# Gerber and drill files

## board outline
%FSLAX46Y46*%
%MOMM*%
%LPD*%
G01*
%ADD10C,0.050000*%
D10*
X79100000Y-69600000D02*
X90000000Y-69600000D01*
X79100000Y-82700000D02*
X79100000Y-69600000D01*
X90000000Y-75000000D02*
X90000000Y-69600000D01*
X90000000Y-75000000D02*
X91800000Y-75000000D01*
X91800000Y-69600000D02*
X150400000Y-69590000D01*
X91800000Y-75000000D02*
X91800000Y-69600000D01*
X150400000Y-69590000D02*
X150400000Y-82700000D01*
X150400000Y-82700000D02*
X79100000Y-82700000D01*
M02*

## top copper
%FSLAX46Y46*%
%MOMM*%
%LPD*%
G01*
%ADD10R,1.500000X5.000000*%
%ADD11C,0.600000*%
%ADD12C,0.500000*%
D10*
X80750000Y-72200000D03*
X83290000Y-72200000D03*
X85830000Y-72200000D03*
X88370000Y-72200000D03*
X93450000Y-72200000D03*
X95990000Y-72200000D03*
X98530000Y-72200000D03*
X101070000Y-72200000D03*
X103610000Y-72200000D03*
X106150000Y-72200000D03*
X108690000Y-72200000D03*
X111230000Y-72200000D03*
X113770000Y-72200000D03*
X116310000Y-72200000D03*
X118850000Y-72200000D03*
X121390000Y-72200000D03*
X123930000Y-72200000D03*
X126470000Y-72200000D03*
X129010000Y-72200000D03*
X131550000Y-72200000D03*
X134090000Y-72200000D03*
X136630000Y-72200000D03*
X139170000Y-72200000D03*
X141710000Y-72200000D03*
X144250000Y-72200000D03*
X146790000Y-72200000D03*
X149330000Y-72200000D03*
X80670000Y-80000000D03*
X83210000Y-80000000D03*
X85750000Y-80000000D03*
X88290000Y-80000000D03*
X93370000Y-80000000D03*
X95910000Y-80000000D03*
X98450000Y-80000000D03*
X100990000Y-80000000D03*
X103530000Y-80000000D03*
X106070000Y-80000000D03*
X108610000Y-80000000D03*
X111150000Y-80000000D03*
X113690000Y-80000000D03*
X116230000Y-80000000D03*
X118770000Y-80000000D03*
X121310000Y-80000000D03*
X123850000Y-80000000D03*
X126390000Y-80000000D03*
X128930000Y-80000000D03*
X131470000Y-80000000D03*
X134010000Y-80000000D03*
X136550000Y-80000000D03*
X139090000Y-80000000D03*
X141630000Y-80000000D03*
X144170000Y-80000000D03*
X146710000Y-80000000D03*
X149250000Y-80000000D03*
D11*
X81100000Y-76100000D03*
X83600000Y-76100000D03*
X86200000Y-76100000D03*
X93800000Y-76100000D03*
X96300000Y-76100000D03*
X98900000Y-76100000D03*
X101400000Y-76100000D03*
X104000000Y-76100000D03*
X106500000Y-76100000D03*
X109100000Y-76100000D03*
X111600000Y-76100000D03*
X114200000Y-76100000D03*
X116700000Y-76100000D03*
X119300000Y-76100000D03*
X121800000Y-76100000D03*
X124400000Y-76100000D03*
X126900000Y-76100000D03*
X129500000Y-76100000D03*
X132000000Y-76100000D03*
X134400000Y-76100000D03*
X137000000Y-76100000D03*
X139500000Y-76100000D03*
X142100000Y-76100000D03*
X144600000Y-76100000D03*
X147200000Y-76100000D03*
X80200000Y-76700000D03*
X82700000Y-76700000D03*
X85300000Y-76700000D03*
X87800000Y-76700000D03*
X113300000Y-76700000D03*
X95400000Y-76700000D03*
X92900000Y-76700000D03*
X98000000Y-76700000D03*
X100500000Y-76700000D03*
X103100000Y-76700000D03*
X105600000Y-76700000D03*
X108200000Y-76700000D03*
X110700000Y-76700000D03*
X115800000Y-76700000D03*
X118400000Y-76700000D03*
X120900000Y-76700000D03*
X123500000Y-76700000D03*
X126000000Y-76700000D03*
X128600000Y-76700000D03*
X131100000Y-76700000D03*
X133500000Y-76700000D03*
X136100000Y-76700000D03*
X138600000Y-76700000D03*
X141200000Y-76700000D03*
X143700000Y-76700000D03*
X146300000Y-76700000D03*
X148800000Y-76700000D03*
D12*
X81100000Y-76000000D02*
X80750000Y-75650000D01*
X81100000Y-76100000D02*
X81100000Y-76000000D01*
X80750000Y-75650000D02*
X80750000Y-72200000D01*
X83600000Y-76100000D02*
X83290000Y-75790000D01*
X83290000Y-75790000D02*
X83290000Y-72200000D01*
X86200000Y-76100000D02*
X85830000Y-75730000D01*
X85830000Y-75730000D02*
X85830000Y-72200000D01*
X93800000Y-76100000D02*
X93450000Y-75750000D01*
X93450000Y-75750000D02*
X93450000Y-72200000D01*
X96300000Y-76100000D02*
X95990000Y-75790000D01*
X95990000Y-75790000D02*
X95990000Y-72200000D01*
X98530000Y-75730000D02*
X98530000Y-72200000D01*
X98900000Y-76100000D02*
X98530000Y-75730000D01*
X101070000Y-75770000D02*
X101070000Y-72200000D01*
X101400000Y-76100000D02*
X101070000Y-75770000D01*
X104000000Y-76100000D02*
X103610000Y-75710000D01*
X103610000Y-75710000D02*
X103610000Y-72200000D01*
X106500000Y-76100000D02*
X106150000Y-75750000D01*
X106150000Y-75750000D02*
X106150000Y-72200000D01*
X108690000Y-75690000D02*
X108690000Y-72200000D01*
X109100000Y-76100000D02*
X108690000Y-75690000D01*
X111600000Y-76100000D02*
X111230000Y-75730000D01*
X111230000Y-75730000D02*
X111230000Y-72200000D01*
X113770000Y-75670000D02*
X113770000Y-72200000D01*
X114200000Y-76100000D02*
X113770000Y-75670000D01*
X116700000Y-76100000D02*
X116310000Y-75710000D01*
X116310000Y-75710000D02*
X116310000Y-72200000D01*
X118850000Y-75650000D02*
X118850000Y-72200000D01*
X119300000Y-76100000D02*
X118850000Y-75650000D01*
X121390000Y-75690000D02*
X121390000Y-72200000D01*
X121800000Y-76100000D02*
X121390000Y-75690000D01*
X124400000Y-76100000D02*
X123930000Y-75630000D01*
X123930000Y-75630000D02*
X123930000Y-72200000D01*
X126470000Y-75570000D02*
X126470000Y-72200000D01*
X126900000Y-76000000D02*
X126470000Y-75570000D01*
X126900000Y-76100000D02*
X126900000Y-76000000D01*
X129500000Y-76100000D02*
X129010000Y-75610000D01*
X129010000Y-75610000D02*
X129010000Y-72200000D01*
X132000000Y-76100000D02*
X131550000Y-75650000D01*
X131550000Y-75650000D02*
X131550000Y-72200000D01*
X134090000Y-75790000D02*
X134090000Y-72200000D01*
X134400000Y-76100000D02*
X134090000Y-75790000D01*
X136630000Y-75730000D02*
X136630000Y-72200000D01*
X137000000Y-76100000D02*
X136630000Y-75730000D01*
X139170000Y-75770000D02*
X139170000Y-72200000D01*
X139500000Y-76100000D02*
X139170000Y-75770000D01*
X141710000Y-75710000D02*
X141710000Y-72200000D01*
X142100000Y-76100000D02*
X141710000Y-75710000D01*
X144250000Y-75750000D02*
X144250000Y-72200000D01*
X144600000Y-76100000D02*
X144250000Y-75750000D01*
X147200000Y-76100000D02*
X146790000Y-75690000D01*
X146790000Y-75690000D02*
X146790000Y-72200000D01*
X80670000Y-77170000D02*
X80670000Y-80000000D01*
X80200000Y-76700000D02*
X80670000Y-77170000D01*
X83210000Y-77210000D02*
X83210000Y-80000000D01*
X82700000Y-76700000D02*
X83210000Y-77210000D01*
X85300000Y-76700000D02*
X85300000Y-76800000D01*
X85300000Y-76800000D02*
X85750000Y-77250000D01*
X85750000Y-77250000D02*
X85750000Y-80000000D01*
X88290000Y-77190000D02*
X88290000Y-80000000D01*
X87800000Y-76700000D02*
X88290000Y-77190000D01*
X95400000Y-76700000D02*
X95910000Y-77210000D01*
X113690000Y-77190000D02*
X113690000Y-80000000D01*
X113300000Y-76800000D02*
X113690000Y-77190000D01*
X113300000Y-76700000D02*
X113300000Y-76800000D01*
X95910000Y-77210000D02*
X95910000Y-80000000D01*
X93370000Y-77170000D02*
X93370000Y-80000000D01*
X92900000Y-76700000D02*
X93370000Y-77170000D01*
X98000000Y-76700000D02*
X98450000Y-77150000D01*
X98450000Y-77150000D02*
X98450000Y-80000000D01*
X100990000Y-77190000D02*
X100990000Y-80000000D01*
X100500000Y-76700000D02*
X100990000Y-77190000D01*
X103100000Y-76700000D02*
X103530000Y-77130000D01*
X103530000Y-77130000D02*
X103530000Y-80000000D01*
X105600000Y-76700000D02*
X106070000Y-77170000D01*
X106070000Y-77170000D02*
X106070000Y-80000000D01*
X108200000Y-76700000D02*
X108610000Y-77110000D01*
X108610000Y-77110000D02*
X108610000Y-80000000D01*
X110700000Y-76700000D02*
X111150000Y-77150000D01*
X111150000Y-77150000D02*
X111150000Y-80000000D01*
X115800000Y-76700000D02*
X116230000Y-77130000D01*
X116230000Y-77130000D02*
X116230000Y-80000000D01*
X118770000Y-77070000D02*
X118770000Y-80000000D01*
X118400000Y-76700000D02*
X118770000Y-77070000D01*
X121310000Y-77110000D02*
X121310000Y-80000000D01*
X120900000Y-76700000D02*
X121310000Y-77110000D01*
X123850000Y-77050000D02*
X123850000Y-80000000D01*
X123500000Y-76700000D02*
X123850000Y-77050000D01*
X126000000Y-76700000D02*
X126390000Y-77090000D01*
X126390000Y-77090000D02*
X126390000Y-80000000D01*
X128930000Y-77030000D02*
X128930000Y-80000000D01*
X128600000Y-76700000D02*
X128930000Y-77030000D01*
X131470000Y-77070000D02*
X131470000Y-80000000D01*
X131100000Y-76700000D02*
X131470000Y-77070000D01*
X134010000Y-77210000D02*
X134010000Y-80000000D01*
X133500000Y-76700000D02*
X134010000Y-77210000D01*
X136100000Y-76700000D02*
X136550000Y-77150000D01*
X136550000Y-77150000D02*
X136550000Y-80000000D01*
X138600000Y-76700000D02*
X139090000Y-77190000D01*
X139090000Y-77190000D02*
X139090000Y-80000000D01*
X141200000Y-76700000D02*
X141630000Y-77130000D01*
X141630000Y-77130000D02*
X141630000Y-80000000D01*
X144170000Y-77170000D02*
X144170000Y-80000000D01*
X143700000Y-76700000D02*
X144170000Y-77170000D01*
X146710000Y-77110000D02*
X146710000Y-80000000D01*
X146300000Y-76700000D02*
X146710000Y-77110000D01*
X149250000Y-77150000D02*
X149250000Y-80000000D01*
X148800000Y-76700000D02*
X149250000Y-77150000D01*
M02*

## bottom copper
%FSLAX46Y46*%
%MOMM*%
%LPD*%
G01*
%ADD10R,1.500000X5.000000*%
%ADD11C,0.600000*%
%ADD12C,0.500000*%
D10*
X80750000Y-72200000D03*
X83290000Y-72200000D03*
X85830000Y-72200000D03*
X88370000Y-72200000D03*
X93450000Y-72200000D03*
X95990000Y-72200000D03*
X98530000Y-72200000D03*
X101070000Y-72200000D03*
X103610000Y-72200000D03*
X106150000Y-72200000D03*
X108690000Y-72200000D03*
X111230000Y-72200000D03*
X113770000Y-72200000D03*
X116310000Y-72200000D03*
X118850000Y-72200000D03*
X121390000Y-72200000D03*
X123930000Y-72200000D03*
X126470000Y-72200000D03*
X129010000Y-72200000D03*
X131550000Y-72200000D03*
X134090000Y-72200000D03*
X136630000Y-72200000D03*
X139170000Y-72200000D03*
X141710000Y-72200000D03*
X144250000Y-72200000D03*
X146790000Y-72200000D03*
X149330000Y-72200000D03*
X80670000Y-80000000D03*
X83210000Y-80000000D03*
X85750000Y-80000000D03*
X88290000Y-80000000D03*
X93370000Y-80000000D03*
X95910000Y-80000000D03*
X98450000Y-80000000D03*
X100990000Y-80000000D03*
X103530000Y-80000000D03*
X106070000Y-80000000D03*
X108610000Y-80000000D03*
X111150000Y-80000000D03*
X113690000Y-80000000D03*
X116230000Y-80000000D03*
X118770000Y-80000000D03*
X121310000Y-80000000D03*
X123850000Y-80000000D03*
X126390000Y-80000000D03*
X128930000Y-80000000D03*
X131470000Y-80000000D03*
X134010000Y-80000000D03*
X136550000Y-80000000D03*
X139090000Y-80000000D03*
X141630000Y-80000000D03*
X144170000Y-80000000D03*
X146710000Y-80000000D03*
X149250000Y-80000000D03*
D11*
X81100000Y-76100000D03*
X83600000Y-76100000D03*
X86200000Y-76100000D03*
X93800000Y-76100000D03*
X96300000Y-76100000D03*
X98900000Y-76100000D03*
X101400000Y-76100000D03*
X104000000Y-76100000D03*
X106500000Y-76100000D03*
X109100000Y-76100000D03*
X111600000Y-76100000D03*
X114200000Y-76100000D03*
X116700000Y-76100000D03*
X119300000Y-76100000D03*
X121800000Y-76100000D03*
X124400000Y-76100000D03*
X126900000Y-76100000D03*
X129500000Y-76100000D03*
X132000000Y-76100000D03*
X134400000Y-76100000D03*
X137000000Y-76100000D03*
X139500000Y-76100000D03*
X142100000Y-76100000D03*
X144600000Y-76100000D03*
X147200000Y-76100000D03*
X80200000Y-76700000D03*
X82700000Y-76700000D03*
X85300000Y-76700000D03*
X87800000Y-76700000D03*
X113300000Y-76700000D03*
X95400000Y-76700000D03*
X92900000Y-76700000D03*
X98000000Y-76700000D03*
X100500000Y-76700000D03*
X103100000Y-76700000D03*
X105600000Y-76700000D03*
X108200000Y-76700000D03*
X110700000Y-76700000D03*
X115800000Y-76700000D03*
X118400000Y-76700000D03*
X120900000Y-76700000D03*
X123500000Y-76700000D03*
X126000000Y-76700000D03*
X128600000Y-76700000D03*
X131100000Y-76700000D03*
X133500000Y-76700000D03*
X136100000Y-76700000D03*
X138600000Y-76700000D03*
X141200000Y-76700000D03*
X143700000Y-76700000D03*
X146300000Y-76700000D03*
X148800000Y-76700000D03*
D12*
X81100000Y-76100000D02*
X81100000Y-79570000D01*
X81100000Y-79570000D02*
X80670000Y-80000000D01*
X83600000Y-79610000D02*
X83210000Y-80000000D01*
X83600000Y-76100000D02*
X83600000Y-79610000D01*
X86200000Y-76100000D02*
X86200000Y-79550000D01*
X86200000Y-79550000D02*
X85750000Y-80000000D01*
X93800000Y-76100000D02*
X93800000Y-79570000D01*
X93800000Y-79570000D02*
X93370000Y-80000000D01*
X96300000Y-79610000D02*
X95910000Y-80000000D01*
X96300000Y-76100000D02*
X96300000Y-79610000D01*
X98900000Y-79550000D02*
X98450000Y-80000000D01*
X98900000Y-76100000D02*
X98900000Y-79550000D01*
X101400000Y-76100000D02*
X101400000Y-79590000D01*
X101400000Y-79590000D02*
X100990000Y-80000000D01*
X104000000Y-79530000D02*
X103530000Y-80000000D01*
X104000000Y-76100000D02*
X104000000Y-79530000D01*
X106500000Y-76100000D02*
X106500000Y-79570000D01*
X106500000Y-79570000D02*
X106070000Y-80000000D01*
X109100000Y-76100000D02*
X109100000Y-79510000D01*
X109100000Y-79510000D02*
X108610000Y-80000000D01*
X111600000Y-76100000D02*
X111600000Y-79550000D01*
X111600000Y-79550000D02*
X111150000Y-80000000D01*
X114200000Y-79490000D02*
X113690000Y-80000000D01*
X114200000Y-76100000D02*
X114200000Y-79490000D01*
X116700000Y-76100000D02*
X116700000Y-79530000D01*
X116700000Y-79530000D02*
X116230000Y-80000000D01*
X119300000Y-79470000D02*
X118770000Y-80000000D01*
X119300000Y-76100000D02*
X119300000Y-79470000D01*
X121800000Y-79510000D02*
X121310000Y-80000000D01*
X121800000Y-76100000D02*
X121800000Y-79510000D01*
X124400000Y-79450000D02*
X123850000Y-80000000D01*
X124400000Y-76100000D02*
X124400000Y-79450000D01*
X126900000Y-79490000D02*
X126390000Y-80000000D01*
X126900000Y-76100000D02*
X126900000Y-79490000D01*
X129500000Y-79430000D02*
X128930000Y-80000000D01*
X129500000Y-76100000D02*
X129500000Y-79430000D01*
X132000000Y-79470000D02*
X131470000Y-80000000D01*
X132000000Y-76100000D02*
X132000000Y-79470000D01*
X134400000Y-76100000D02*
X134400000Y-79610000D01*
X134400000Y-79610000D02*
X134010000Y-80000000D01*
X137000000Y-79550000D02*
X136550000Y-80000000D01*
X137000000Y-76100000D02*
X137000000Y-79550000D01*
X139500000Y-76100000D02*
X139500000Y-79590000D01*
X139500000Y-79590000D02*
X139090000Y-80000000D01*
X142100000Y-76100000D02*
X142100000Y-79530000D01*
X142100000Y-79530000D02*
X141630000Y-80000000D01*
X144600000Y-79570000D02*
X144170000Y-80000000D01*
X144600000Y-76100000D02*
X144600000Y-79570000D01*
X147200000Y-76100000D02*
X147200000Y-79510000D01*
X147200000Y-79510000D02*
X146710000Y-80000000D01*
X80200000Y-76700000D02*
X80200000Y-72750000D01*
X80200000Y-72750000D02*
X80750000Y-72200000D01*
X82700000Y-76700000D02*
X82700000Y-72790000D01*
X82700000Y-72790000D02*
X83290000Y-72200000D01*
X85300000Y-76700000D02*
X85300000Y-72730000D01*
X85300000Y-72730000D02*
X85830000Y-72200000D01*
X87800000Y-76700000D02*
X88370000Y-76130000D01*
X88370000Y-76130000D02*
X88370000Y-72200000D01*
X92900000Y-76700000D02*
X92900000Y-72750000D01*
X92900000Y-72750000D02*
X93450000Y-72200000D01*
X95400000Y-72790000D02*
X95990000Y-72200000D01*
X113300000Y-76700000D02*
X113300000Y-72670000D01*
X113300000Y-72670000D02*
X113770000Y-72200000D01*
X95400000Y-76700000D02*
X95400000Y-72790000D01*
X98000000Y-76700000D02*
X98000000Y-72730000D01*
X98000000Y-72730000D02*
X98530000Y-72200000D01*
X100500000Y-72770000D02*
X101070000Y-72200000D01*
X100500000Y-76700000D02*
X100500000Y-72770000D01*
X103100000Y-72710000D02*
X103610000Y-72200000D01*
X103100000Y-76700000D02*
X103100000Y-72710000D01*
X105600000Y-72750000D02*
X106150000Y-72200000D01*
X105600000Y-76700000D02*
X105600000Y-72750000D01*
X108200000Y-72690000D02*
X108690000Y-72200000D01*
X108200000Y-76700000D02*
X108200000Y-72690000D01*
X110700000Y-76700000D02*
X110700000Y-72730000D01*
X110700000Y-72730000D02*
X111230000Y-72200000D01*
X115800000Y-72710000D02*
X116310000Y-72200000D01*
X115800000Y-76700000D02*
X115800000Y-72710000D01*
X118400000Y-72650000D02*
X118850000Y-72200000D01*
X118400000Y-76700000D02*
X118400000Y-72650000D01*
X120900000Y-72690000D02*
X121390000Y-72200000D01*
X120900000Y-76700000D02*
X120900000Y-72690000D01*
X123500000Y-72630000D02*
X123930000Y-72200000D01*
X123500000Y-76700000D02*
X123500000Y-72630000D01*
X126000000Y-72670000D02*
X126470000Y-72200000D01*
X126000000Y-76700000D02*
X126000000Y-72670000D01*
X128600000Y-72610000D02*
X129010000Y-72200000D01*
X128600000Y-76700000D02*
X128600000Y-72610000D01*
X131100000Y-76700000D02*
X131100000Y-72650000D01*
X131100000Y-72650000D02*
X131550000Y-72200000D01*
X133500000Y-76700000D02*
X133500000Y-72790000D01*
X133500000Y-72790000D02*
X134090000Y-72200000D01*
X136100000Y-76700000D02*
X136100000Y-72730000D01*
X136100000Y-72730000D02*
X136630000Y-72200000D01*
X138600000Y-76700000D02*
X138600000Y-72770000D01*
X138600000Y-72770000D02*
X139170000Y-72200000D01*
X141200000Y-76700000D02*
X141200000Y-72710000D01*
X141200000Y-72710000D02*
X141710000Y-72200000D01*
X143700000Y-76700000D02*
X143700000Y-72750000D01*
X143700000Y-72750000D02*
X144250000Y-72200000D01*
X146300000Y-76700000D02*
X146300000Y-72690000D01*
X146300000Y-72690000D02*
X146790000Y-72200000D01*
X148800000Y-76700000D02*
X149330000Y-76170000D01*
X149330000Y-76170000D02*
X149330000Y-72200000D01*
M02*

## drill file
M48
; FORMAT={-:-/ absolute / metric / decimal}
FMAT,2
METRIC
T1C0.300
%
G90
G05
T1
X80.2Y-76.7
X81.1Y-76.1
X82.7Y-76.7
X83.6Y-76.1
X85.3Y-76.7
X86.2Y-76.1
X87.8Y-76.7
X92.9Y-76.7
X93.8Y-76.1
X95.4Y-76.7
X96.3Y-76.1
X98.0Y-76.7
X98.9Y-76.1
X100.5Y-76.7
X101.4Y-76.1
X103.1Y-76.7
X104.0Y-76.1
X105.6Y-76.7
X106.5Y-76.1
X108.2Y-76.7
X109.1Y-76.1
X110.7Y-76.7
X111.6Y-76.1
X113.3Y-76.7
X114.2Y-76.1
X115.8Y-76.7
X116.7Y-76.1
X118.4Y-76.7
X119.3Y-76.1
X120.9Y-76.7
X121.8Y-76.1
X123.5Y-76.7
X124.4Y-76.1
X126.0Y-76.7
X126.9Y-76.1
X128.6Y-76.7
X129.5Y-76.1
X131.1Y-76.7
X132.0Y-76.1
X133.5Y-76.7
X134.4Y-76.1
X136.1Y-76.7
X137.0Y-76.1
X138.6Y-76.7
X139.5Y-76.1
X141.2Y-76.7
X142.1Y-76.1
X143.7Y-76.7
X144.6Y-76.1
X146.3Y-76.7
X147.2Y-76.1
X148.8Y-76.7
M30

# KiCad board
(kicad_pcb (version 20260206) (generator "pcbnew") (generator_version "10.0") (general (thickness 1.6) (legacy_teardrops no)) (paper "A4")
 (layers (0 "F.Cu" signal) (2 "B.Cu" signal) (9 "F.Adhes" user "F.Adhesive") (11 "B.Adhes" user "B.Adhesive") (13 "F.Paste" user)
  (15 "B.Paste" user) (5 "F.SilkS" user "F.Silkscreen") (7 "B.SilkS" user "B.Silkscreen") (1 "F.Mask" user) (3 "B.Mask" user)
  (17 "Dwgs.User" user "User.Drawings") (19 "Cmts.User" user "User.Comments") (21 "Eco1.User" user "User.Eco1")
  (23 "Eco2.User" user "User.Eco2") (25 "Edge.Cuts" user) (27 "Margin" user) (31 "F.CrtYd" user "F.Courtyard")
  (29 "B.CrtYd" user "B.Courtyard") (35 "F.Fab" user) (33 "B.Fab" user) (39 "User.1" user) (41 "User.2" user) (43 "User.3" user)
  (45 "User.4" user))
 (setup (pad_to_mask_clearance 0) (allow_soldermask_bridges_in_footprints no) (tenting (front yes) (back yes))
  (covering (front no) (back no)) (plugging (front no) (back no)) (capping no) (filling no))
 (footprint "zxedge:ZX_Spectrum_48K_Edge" (layer "F.Cu") (at 115.04 74.7)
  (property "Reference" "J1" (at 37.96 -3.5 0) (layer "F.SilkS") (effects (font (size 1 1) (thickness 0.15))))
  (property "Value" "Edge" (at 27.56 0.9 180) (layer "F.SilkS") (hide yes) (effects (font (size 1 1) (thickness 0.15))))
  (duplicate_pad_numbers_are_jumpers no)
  (pad "A1" smd rect (at -34.29 -2.5) (size 1.5 5) (layers "F.Cu" "F.Mask") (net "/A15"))
  (pad "A2" smd rect (at -31.75 -2.5) (size 1.5 5) (layers "F.Cu" "F.Mask") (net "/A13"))
  (pad "A3" smd rect (at -29.21 -2.5) (size 1.5 5) (layers "F.Cu" "F.Mask") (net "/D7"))
  (pad "A4" smd rect (at -26.67 -2.5) (size 1.5 5) (layers "F.Cu" "F.Mask") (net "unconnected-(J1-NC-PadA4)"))
  (pad "A6" smd rect (at -21.59 -2.5) (size 1.5 5) (layers "F.Cu" "F.Mask") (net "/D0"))
  (pad "A7" smd rect (at -19.05 -2.5) (size 1.5 5) (layers "F.Cu" "F.Mask") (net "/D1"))
  (pad "A8" smd rect (at -16.51 -2.5) (size 1.5 5) (layers "F.Cu" "F.Mask") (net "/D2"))
  (pad "A9" smd rect (at -13.97 -2.5) (size 1.5 5) (layers "F.Cu" "F.Mask") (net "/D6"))
  (pad "A10" smd rect (at -11.43 -2.5) (size 1.5 5) (layers "F.Cu" "F.Mask") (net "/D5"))
  (pad "A11" smd rect (at -8.89 -2.5) (size 1.5 5) (layers "F.Cu" "F.Mask") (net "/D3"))
  (pad "A12" smd rect (at -6.35 -2.5) (size 1.5 5) (layers "F.Cu" "F.Mask") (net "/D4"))
  (pad "A13" smd rect (at -3.81 -2.5) (size 1.5 5) (layers "F.Cu" "F.Mask") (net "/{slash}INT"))
  (pad "A14" smd rect (at -1.27 -2.5) (size 1.5 5) (layers "F.Cu" "F.Mask") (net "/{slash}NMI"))
  (pad "A15" smd rect (at 1.27 -2.5) (size 1.5 5) (layers "F.Cu" "F.Mask") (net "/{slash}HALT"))
  (pad "A16" smd rect (at 3.81 -2.5) (size 1.5 5) (layers "F.Cu" "F.Mask") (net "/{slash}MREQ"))
  (pad "A17" smd rect (at 6.35 -2.5) (size 1.5 5) (layers "F.Cu" "F.Mask") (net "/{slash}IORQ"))
  (pad "A18" smd rect (at 8.89 -2.5) (size 1.5 5) (layers "F.Cu" "F.Mask") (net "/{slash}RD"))
  (pad "A19" smd rect (at 11.43 -2.5) (size 1.5 5) (layers "F.Cu" "F.Mask") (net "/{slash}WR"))
  (pad "A20" smd rect (at 13.97 -2.5) (size 1.5 5) (layers "F.Cu" "F.Mask") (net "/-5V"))
  (pad "A21" smd rect (at 16.51 -2.5) (size 1.5 5) (layers "F.Cu" "F.Mask") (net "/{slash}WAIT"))
  (pad "A22" smd rect (at 19.05 -2.5) (size 1.5 5) (layers "F.Cu" "F.Mask") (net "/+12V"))
  (pad "A23" smd rect (at 21.59 -2.5) (size 1.5 5) (layers "F.Cu" "F.Mask") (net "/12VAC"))
  (pad "A24" smd rect (at 24.13 -2.5) (size 1.5 5) (layers "F.Cu" "F.Mask") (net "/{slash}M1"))
  (pad "A25" smd rect (at 26.67 -2.5) (size 1.5 5) (layers "F.Cu" "F.Mask") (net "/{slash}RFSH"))
  (pad "A26" smd rect (at 29.21 -2.5) (size 1.5 5) (layers "F.Cu" "F.Mask") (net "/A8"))
  (pad "A27" smd rect (at 31.75 -2.5) (size 1.5 5) (layers "F.Cu" "F.Mask") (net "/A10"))
  (pad "A28" smd rect (at 34.29 -2.5) (size 1.5 5) (layers "F.Cu" "F.Mask") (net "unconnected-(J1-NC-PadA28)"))
  (pad "B1" smd rect (at -34.29 -2.5) (size 1.5 5) (layers "B.Cu" "B.Mask") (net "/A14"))
  (pad "B2" smd rect (at -31.75 -2.5) (size 1.5 5) (layers "B.Cu" "B.Mask") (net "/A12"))
  (pad "B3" smd rect (at -29.21 -2.5) (size 1.5 5) (layers "B.Cu" "B.Mask") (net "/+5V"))
  (pad "B4" smd rect (at -26.67 -2.5) (size 1.5 5) (layers "B.Cu" "B.Mask") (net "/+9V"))
  (pad "B6" smd rect (at -21.59 -2.5) (size 1.5 5) (layers "B.Cu" "B.Mask") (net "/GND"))
  (pad "B7" smd rect (at -19.05 -2.5) (size 1.5 5) (layers "B.Cu" "B.Mask") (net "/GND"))
  (pad "B8" smd rect (at -16.51 -2.5) (size 1.5 5) (layers "B.Cu" "B.Mask") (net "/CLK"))
  (pad "B9" smd rect (at -13.97 -2.5) (size 1.5 5) (layers "B.Cu" "B.Mask") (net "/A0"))
  (pad "B10" smd rect (at -11.43 -2.5) (size 1.5 5) (layers "B.Cu" "B.Mask") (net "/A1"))
  (pad "B11" smd rect (at -8.89 -2.5) (size 1.5 5) (layers "B.Cu" "B.Mask") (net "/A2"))
  (pad "B12" smd rect (at -6.35 -2.5) (size 1.5 5) (layers "B.Cu" "B.Mask") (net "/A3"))
  (pad "B13" smd rect (at -3.81 -2.5) (size 1.5 5) (layers "B.Cu" "B.Mask") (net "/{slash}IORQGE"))
  (pad "B14" smd rect (at -1.27 -2.5) (size 1.5 5) (layers "B.Cu" "B.Mask") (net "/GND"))
  (pad "B15" smd rect (at 1.27 -2.5) (size 1.5 5) (layers "B.Cu" "B.Mask") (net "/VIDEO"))
  (pad "B16" smd rect (at 3.81 -2.5) (size 1.5 5) (layers "B.Cu" "B.Mask") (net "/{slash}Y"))
  (pad "B17" smd rect (at 6.35 -2.5) (size 1.5 5) (layers "B.Cu" "B.Mask") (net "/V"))
  (pad "B18" smd rect (at 8.89 -2.5) (size 1.5 5) (layers "B.Cu" "B.Mask") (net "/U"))
  (pad "B19" smd rect (at 11.43 -2.5) (size 1.5 5) (layers "B.Cu" "B.Mask") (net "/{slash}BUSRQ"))
  (pad "B20" smd rect (at 13.97 -2.5) (size 1.5 5) (layers "B.Cu" "B.Mask") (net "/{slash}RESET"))
  (pad "B21" smd rect (at 16.51 -2.5) (size 1.5 5) (layers "B.Cu" "B.Mask") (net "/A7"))
  (pad "B22" smd rect (at 19.05 -2.5) (size 1.5 5) (layers "B.Cu" "B.Mask") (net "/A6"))
  (pad "B23" smd rect (at 21.59 -2.5) (size 1.5 5) (layers "B.Cu" "B.Mask") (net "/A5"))
  (pad "B24" smd rect (at 24.13 -2.5) (size 1.5 5) (layers "B.Cu" "B.Mask") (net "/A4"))
  (pad "B25" smd rect (at 26.67 -2.5) (size 1.5 5) (layers "B.Cu" "B.Mask") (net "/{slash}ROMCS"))
  (pad "B26" smd rect (at 29.21 -2.5) (size 1.5 5) (layers "B.Cu" "B.Mask") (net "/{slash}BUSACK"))
  (pad "B27" smd rect (at 31.75 -2.5) (size 1.5 5) (layers "B.Cu" "B.Mask") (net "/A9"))
  (pad "B28" smd rect (at 34.29 -2.5) (size 1.5 5) (layers "B.Cu" "B.Mask") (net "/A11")))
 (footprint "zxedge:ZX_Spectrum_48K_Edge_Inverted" (layer "B.Cu") (at 114.96 77.5)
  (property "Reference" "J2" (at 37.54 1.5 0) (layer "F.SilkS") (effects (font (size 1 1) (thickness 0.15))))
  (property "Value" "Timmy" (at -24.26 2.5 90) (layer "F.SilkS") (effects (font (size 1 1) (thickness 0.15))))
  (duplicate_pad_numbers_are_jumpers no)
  (pad "A1" smd rect (at -34.29 2.5) (size 1.5 5) (layers "F.Cu" "F.Mask") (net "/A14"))
  (pad "A2" smd rect (at -31.75 2.5) (size 1.5 5) (layers "F.Cu" "F.Mask") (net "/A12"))
  (pad "A3" smd rect (at -29.21 2.5) (size 1.5 5) (layers "F.Cu" "F.Mask") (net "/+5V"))
  (pad "A4" smd rect (at -26.67 2.5) (size 1.5 5) (layers "F.Cu" "F.Mask") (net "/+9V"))
  (pad "A6" smd rect (at -21.59 2.5) (size 1.5 5) (layers "F.Cu" "F.Mask") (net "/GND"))
  (pad "A7" smd rect (at -19.05 2.5) (size 1.5 5) (layers "F.Cu" "F.Mask") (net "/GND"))
  (pad "A8" smd rect (at -16.51 2.5) (size 1.5 5) (layers "F.Cu" "F.Mask") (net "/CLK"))
  (pad "A9" smd rect (at -13.97 2.5) (size 1.5 5) (layers "F.Cu" "F.Mask") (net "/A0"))
  (pad "A10" smd rect (at -11.43 2.5) (size 1.5 5) (layers "F.Cu" "F.Mask") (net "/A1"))
  (pad "A11" smd rect (at -8.89 2.5) (size 1.5 5) (layers "F.Cu" "F.Mask") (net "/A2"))
  (pad "A12" smd rect (at -6.35 2.5) (size 1.5 5) (layers "F.Cu" "F.Mask") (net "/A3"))
  (pad "A13" smd rect (at -3.81 2.5) (size 1.5 5) (layers "F.Cu" "F.Mask") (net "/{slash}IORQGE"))
  (pad "A14" smd rect (at -1.27 2.5) (size 1.5 5) (layers "F.Cu" "F.Mask") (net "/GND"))
  (pad "A15" smd rect (at 1.27 2.5) (size 1.5 5) (layers "F.Cu" "F.Mask") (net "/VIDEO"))
  (pad "A16" smd rect (at 3.81 2.5) (size 1.5 5) (layers "F.Cu" "F.Mask") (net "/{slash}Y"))
  (pad "A17" smd rect (at 6.35 2.5) (size 1.5 5) (layers "F.Cu" "F.Mask") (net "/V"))
  (pad "A18" smd rect (at 8.89 2.5) (size 1.5 5) (layers "F.Cu" "F.Mask") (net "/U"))
  (pad "A19" smd rect (at 11.43 2.5) (size 1.5 5) (layers "F.Cu" "F.Mask") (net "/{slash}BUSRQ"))
  (pad "A20" smd rect (at 13.97 2.5) (size 1.5 5) (layers "F.Cu" "F.Mask") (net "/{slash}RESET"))
  (pad "A21" smd rect (at 16.51 2.5) (size 1.5 5) (layers "F.Cu" "F.Mask") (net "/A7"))
  (pad "A22" smd rect (at 19.05 2.5) (size 1.5 5) (layers "F.Cu" "F.Mask") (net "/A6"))
  (pad "A23" smd rect (at 21.59 2.5) (size 1.5 5) (layers "F.Cu" "F.Mask") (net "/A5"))
  (pad "A24" smd rect (at 24.13 2.5) (size 1.5 5) (layers "F.Cu" "F.Mask") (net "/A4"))
  (pad "A25" smd rect (at 26.67 2.5) (size 1.5 5) (layers "F.Cu" "F.Mask") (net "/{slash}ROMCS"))
  (pad "A26" smd rect (at 29.21 2.5) (size 1.5 5) (layers "F.Cu" "F.Mask") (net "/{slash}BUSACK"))
  (pad "A27" smd rect (at 31.75 2.5) (size 1.5 5) (layers "F.Cu" "F.Mask") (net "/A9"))
  (pad "A28" smd rect (at 34.29 2.5) (size 1.5 5) (layers "F.Cu" "F.Mask") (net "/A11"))
  (pad "B1" smd rect (at -34.29 2.5) (size 1.5 5) (layers "B.Cu" "B.Mask") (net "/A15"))
  (pad "B2" smd rect (at -31.75 2.5) (size 1.5 5) (layers "B.Cu" "B.Mask") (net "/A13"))
  (pad "B3" smd rect (at -29.21 2.5) (size 1.5 5) (layers "B.Cu" "B.Mask") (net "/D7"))
  (pad "B4" smd rect (at -26.67 2.5) (size 1.5 5) (layers "B.Cu" "B.Mask") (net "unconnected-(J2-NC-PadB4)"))
  (pad "B6" smd rect (at -21.59 2.5) (size 1.5 5) (layers "B.Cu" "B.Mask") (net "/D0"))
  (pad "B7" smd rect (at -19.05 2.5) (size 1.5 5) (layers "B.Cu" "B.Mask") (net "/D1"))
  (pad "B8" smd rect (at -16.51 2.5) (size 1.5 5) (layers "B.Cu" "B.Mask") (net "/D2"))
  (pad "B9" smd rect (at -13.97 2.5) (size 1.5 5) (layers "B.Cu" "B.Mask") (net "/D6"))
  (pad "B10" smd rect (at -11.43 2.5) (size 1.5 5) (layers "B.Cu" "B.Mask") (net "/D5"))
  (pad "B11" smd rect (at -8.89 2.5) (size 1.5 5) (layers "B.Cu" "B.Mask") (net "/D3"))
  (pad "B12" smd rect (at -6.35 2.5) (size 1.5 5) (layers "B.Cu" "B.Mask") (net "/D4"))
  (pad "B13" smd rect (at -3.81 2.5) (size 1.5 5) (layers "B.Cu" "B.Mask") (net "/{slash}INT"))
  (pad "B14" smd rect (at -1.27 2.5) (size 1.5 5) (layers "B.Cu" "B.Mask") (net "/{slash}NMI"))
  (pad "B15" smd rect (at 1.27 2.5) (size 1.5 5) (layers "B.Cu" "B.Mask") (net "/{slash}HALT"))
  (pad "B16" smd rect (at 3.81 2.5) (size 1.5 5) (layers "B.Cu" "B.Mask") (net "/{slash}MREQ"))
  (pad "B17" smd rect (at 6.35 2.5) (size 1.5 5) (layers "B.Cu" "B.Mask") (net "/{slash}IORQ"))
  (pad "B18" smd rect (at 8.89 2.5) (size 1.5 5) (layers "B.Cu" "B.Mask") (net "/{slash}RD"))
  (pad "B19" smd rect (at 11.43 2.5) (size 1.5 5) (layers "B.Cu" "B.Mask") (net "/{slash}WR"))
  (pad "B20" smd rect (at 13.97 2.5) (size 1.5 5) (layers "B.Cu" "B.Mask") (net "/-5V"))
  (pad "B21" smd rect (at 16.51 2.5) (size 1.5 5) (layers "B.Cu" "B.Mask") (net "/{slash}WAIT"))
  (pad "B22" smd rect (at 19.05 2.5) (size 1.5 5) (layers "B.Cu" "B.Mask") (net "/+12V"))
  (pad "B23" smd rect (at 21.59 2.5) (size 1.5 5) (layers "B.Cu" "B.Mask") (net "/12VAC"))
  (pad "B24" smd rect (at 24.13 2.5) (size 1.5 5) (layers "B.Cu" "B.Mask") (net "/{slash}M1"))
  (pad "B25" smd rect (at 26.67 2.5) (size 1.5 5) (layers "B.Cu" "B.Mask") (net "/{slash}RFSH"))
  (pad "B26" smd rect (at 29.21 2.5) (size 1.5 5) (layers "B.Cu" "B.Mask") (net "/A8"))
  (pad "B27" smd rect (at 31.75 2.5) (size 1.5 5) (layers "B.Cu" "B.Mask") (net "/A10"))
  (pad "B28" smd rect (at 34.29 2.5) (size 1.5 5) (layers "B.Cu" "B.Mask") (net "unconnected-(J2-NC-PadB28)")))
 (gr_line (start 79.1 69.6) (end 90 69.6) (stroke (width 0.05) (type default)) (layer "Edge.Cuts"))
 (gr_line (start 79.1 82.7) (end 79.1 69.6) (stroke (width 0.05) (type default)) (layer "Edge.Cuts"))
 (gr_line (start 90 75) (end 90 69.6) (stroke (width 0.05) (type default)) (layer "Edge.Cuts"))
 (gr_line (start 90 75) (end 91.8 75) (stroke (width 0.05) (type default)) (layer "Edge.Cuts"))
 (gr_line (start 91.8 69.6) (end 150.4 69.59) (stroke (width 0.05) (type default)) (layer "Edge.Cuts"))
 (gr_line (start 91.8 75) (end 91.8 69.6) (stroke (width 0.05) (type default)) (layer "Edge.Cuts"))
 (gr_line (start 150.4 69.59) (end 150.4 82.7) (stroke (width 0.05) (type default)) (layer "Edge.Cuts"))
 (gr_line (start 150.4 82.7) (end 79.1 82.7) (stroke (width 0.05) (type default)) (layer "Edge.Cuts"))
 (segment (start 81.1 76) (end 80.75 75.65) (width 0.5) (layer "F.Cu") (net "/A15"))
 (segment (start 81.1 76.1) (end 81.1 76) (width 0.5) (layer "F.Cu") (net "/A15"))
 (segment (start 80.75 75.65) (end 80.75 72.2) (width 0.5) (layer "F.Cu") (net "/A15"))
 (via (at 81.1 76.1) (size 0.6) (drill 0.3) (layers "F.Cu" "B.Cu") (free yes) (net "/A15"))
 (segment (start 81.1 76.1) (end 81.1 79.57) (width 0.5) (layer "B.Cu") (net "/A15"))
 (segment (start 81.1 79.57) (end 80.67 80) (width 0.5) (layer "B.Cu") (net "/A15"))
 (segment (start 83.6 76.1) (end 83.29 75.79) (width 0.5) (layer "F.Cu") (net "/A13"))
 (segment (start 83.29 75.79) (end 83.29 72.2) (width 0.5) (layer "F.Cu") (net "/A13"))
 (via (at 83.6 76.1) (size 0.6) (drill 0.3) (layers "F.Cu" "B.Cu") (free yes) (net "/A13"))
 (segment (start 83.6 79.61) (end 83.21 80) (width 0.5) (layer "B.Cu") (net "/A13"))
 (segment (start 83.6 76.1) (end 83.6 79.61) (width 0.5) (layer "B.Cu") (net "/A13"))
 (segment (start 86.2 76.1) (end 85.83 75.73) (width 0.5) (layer "F.Cu") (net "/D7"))
 (segment (start 85.83 75.73) (end 85.83 72.2) (width 0.5) (layer "F.Cu") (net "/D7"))
 (via (at 86.2 76.1) (size 0.6) (drill 0.3) (layers "F.Cu" "B.Cu") (free yes) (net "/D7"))
 (segment (start 86.2 76.1) (end 86.2 79.55) (width 0.5) (layer "B.Cu") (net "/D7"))
 (segment (start 86.2 79.55) (end 85.75 80) (width 0.5) (layer "B.Cu") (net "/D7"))
 (segment (start 93.8 76.1) (end 93.45 75.75) (width 0.5) (layer "F.Cu") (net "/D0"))
 (segment (start 93.45 75.75) (end 93.45 72.2) (width 0.5) (layer "F.Cu") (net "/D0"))
 (via (at 93.8 76.1) (size 0.6) (drill 0.3) (layers "F.Cu" "B.Cu") (free yes) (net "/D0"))
 (segment (start 93.8 76.1) (end 93.8 79.57) (width 0.5) (layer "B.Cu") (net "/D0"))
 (segment (start 93.8 79.57) (end 93.37 80) (width 0.5) (layer "B.Cu") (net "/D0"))
 (segment (start 96.3 76.1) (end 95.99 75.79) (width 0.5) (layer "F.Cu") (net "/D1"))
 (segment (start 95.99 75.79) (end 95.99 72.2) (width 0.5) (layer "F.Cu") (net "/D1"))
 (via (at 96.3 76.1) (size 0.6) (drill 0.3) (layers "F.Cu" "B.Cu") (free yes) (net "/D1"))
 (segment (start 96.3 79.61) (end 95.91 80) (width 0.5) (layer "B.Cu") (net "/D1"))
 (segment (start 96.3 76.1) (end 96.3 79.61) (width 0.5) (layer "B.Cu") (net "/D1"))
 (segment (start 98.53 75.73) (end 98.53 72.2) (width 0.5) (layer "F.Cu") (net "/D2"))
 (segment (start 98.9 76.1) (end 98.53 75.73) (width 0.5) (layer "F.Cu") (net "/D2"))
 (via (at 98.9 76.1) (size 0.6) (drill 0.3) (layers "F.Cu" "B.Cu") (free yes) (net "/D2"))
 (segment (start 98.9 79.55) (end 98.45 80) (width 0.5) (layer "B.Cu") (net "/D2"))
 (segment (start 98.9 76.1) (end 98.9 79.55) (width 0.5) (layer "B.Cu") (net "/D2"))
 (segment (start 101.07 75.77) (end 101.07 72.2) (width 0.5) (layer "F.Cu") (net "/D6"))
 (segment (start 101.4 76.1) (end 101.07 75.77) (width 0.5) (layer "F.Cu") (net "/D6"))
 (via (at 101.4 76.1) (size 0.6) (drill 0.3) (layers "F.Cu" "B.Cu") (free yes) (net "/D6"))
 (segment (start 101.4 76.1) (end 101.4 79.59) (width 0.5) (layer "B.Cu") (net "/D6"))
 (segment (start 101.4 79.59) (end 100.99 80) (width 0.5) (layer "B.Cu") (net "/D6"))
 (segment (start 104 76.1) (end 103.61 75.71) (width 0.5) (layer "F.Cu") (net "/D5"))
 (segment (start 103.61 75.71) (end 103.61 72.2) (width 0.5) (layer "F.Cu") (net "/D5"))
 (via (at 104 76.1) (size 0.6) (drill 0.3) (layers "F.Cu" "B.Cu") (free yes) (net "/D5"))
 (segment (start 104 79.53) (end 103.53 80) (width 0.5) (layer "B.Cu") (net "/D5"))
 (segment (start 104 76.1) (end 104 79.53) (width 0.5) (layer "B.Cu") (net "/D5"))
 (segment (start 106.5 76.1) (end 106.15 75.75) (width 0.5) (layer "F.Cu") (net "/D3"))
 (segment (start 106.15 75.75) (end 106.15 72.2) (width 0.5) (layer "F.Cu") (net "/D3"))
 (via (at 106.5 76.1) (size 0.6) (drill 0.3) (layers "F.Cu" "B.Cu") (free yes) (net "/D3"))
 (segment (start 106.5 76.1) (end 106.5 79.57) (width 0.5) (layer "B.Cu") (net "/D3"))
 (segment (start 106.5 79.57) (end 106.07 80) (width 0.5) (layer "B.Cu") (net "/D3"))
 (segment (start 108.69 75.69) (end 108.69 72.2) (width 0.5) (layer "F.Cu") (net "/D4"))
 (segment (start 109.1 76.1) (end 108.69 75.69) (width 0.5) (layer "F.Cu") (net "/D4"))
 (via (at 109.1 76.1) (size 0.6) (drill 0.3) (layers "F.Cu" "B.Cu") (free yes) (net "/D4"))
 (segment (start 109.1 76.1) (end 109.1 79.51) (width 0.5) (layer "B.Cu") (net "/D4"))
 (segment (start 109.1 79.51) (end 108.61 80) (width 0.5) (layer "B.Cu") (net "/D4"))
 (segment (start 111.6 76.1) (end 111.23 75.73) (width 0.5) (layer "F.Cu") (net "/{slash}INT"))
 (segment (start 111.23 75.73) (end 111.23 72.2) (width 0.5) (layer "F.Cu") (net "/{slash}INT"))
 (via (at 111.6 76.1) (size 0.6) (drill 0.3) (layers "F.Cu" "B.Cu") (free yes) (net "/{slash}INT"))
 (segment (start 111.6 76.1) (end 111.6 79.55) (width 0.5) (layer "B.Cu") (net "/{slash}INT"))
 (segment (start 111.6 79.55) (end 111.15 80) (width 0.5) (layer "B.Cu") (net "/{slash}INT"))
 (segment (start 113.77 75.67) (end 113.77 72.2) (width 0.5) (layer "F.Cu") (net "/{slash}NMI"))
 (segment (start 114.2 76.1) (end 113.77 75.67) (width 0.5) (layer "F.Cu") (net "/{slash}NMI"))
 (via (at 114.2 76.1) (size 0.6) (drill 0.3) (layers "F.Cu" "B.Cu") (free yes) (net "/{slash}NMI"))
 (segment (start 114.2 79.49) (end 113.69 80) (width 0.5) (layer "B.Cu") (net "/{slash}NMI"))
 (segment (start 114.2 76.1) (end 114.2 79.49) (width 0.5) (layer "B.Cu") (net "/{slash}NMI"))
 (segment (start 116.7 76.1) (end 116.31 75.71) (width 0.5) (layer "F.Cu") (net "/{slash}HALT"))
 (segment (start 116.31 75.71) (end 116.31 72.2) (width 0.5) (layer "F.Cu") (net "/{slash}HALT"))
 (via (at 116.7 76.1) (size 0.6) (drill 0.3) (layers "F.Cu" "B.Cu") (free yes) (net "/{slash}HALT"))
 (segment (start 116.7 76.1) (end 116.7 79.53) (width 0.5) (layer "B.Cu") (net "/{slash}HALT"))
 (segment (start 116.7 79.53) (end 116.23 80) (width 0.5) (layer "B.Cu") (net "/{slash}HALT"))
 (segment (start 118.85 75.65) (end 118.85 72.2) (width 0.5) (layer "F.Cu") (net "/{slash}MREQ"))
 (segment (start 119.3 76.1) (end 118.85 75.65) (width 0.5) (layer "F.Cu") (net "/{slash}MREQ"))
 (via (at 119.3 76.1) (size 0.6) (drill 0.3) (layers "F.Cu" "B.Cu") (free yes) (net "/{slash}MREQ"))
 (segment (start 119.3 79.47) (end 118.77 80) (width 0.5) (layer "B.Cu") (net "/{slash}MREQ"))
 (segment (start 119.3 76.1) (end 119.3 79.47) (width 0.5) (layer "B.Cu") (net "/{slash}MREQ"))
 (segment (start 121.39 75.69) (end 121.39 72.2) (width 0.5) (layer "F.Cu") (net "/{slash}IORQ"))
 (segment (start 121.8 76.1) (end 121.39 75.69) (width 0.5) (layer "F.Cu") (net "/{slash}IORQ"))
 (via (at 121.8 76.1) (size 0.6) (drill 0.3) (layers "F.Cu" "B.Cu") (free yes) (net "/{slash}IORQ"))
 (segment (start 121.8 79.51) (end 121.31 80) (width 0.5) (layer "B.Cu") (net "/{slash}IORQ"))
 (segment (start 121.8 76.1) (end 121.8 79.51) (width 0.5) (layer "B.Cu") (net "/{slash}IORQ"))
 (segment (start 124.4 76.1) (end 123.93 75.63) (width 0.5) (layer "F.Cu") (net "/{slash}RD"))
 (segment (start 123.93 75.63) (end 123.93 72.2) (width 0.5) (layer "F.Cu") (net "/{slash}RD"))
 (via (at 124.4 76.1) (size 0.6) (drill 0.3) (layers "F.Cu" "B.Cu") (free yes) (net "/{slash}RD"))
 (segment (start 124.4 79.45) (end 123.85 80) (width 0.5) (layer "B.Cu") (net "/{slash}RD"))
 (segment (start 124.4 76.1) (end 124.4 79.45) (width 0.5) (layer "B.Cu") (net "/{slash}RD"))
 (segment (start 126.47 75.57) (end 126.47 72.2) (width 0.5) (layer "F.Cu") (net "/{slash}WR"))
 (segment (start 126.9 76) (end 126.47 75.57) (width 0.5) (layer "F.Cu") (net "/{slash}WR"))
 (segment (start 126.9 76.1) (end 126.9 76) (width 0.5) (layer "F.Cu") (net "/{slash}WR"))
 (via (at 126.9 76.1) (size 0.6) (drill 0.3) (layers "F.Cu" "B.Cu") (free yes) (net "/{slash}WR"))
 (segment (start 126.9 79.49) (end 126.39 80) (width 0.5) (layer "B.Cu") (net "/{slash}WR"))
 (segment (start 126.9 76.1) (end 126.9 79.49) (width 0.5) (layer "B.Cu") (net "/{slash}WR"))
 (segment (start 129.5 76.1) (end 129.01 75.61) (width 0.5) (layer "F.Cu") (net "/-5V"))
 (segment (start 129.01 75.61) (end 129.01 72.2) (width 0.5) (layer "F.Cu") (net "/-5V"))
 (via (at 129.5 76.1) (size 0.6) (drill 0.3) (layers "F.Cu" "B.Cu") (free yes) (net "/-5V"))
 (segment (start 129.5 79.43) (end 128.93 80) (width 0.5) (layer "B.Cu") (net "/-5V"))
 (segment (start 129.5 76.1) (end 129.5 79.43) (width 0.5) (layer "B.Cu") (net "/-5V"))
 (segment (start 132 76.1) (end 131.55 75.65) (width 0.5) (layer "F.Cu") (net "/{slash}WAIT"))
 (segment (start 131.55 75.65) (end 131.55 72.2) (width 0.5) (layer "F.Cu") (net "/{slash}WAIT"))
 (via (at 132 76.1) (size 0.6) (drill 0.3) (layers "F.Cu" "B.Cu") (free yes) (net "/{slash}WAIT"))
 (segment (start 132 79.47) (end 131.47 80) (width 0.5) (layer "B.Cu") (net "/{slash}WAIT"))
 (segment (start 132 76.1) (end 132 79.47) (width 0.5) (layer "B.Cu") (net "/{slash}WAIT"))
 (segment (start 134.09 75.79) (end 134.09 72.2) (width 0.5) (layer "F.Cu") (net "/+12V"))
 (segment (start 134.4 76.1) (end 134.09 75.79) (width 0.5) (layer "F.Cu") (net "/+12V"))
 (via (at 134.4 76.1) (size 0.6) (drill 0.3) (layers "F.Cu" "B.Cu") (free yes) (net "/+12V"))
 (segment (start 134.4 76.1) (end 134.4 79.61) (width 0.5) (layer "B.Cu") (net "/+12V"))
 (segment (start 134.4 79.61) (end 134.01 80) (width 0.5) (layer "B.Cu") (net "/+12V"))
 (segment (start 136.63 75.73) (end 136.63 72.2) (width 0.5) (layer "F.Cu") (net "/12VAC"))
 (segment (start 137 76.1) (end 136.63 75.73) (width 0.5) (layer "F.Cu") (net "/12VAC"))
 (via (at 137 76.1) (size 0.6) (drill 0.3) (layers "F.Cu" "B.Cu") (free yes) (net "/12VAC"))
 (segment (start 137 79.55) (end 136.55 80) (width 0.5) (layer "B.Cu") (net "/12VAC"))
 (segment (start 137 76.1) (end 137 79.55) (width 0.5) (layer "B.Cu") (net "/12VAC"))
 (segment (start 139.17 75.77) (end 139.17 72.2) (width 0.5) (layer "F.Cu") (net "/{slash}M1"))
 (segment (start 139.5 76.1) (end 139.17 75.77) (width 0.5) (layer "F.Cu") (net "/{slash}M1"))
 (via (at 139.5 76.1) (size 0.6) (drill 0.3) (layers "F.Cu" "B.Cu") (free yes) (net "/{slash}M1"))
 (segment (start 139.5 76.1) (end 139.5 79.59) (width 0.5) (layer "B.Cu") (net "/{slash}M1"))
 (segment (start 139.5 79.59) (end 139.09 80) (width 0.5) (layer "B.Cu") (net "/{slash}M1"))
 (segment (start 141.71 75.71) (end 141.71 72.2) (width 0.5) (layer "F.Cu") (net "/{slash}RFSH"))
 (segment (start 142.1 76.1) (end 141.71 75.71) (width 0.5) (layer "F.Cu") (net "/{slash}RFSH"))
 (via (at 142.1 76.1) (size 0.6) (drill 0.3) (layers "F.Cu" "B.Cu") (free yes) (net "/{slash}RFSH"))
 (segment (start 142.1 76.1) (end 142.1 79.53) (width 0.5) (layer "B.Cu") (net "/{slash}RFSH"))
 (segment (start 142.1 79.53) (end 141.63 80) (width 0.5) (layer "B.Cu") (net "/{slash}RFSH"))
 (segment (start 144.25 75.75) (end 144.25 72.2) (width 0.5) (layer "F.Cu") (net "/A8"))
 (segment (start 144.6 76.1) (end 144.25 75.75) (width 0.5) (layer "F.Cu") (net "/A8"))
 (via (at 144.6 76.1) (size 0.6) (drill 0.3) (layers "F.Cu" "B.Cu") (free yes) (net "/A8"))
 (segment (start 144.6 79.57) (end 144.17 80) (width 0.5) (layer "B.Cu") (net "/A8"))
 (segment (start 144.6 76.1) (end 144.6 79.57) (width 0.5) (layer "B.Cu") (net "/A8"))
 (segment (start 147.2 76.1) (end 146.79 75.69) (width 0.5) (layer "F.Cu") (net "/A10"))
 (segment (start 146.79 75.69) (end 146.79 72.2) (width 0.5) (layer "F.Cu") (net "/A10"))
 (via (at 147.2 76.1) (size 0.6) (drill 0.3) (layers "F.Cu" "B.Cu") (free yes) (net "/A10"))
 (segment (start 147.2 76.1) (end 147.2 79.51) (width 0.5) (layer "B.Cu") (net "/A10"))
 (segment (start 147.2 79.51) (end 146.71 80) (width 0.5) (layer "B.Cu") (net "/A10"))
 (segment (start 80.67 77.17) (end 80.67 80) (width 0.5) (layer "F.Cu") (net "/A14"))
 (segment (start 80.2 76.7) (end 80.67 77.17) (width 0.5) (layer "F.Cu") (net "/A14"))
 (via (at 80.2 76.7) (size 0.6) (drill 0.3) (layers "F.Cu" "B.Cu") (free yes) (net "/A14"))
 (segment (start 80.2 76.7) (end 80.2 72.75) (width 0.5) (layer "B.Cu") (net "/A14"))
 (segment (start 80.2 72.75) (end 80.75 72.2) (width 0.5) (layer "B.Cu") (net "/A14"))
 (segment (start 83.21 77.21) (end 83.21 80) (width 0.5) (layer "F.Cu") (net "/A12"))
 (segment (start 82.7 76.7) (end 83.21 77.21) (width 0.5) (layer "F.Cu") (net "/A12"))
 (via (at 82.7 76.7) (size 0.6) (drill 0.3) (layers "F.Cu" "B.Cu") (free yes) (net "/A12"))
 (segment (start 82.7 76.7) (end 82.7 72.79) (width 0.5) (layer "B.Cu") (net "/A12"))
 (segment (start 82.7 72.79) (end 83.29 72.2) (width 0.5) (layer "B.Cu") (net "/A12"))
 (segment (start 85.3 76.7) (end 85.3 76.8) (width 0.5) (layer "F.Cu") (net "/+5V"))
 (segment (start 85.3 76.8) (end 85.75 77.25) (width 0.5) (layer "F.Cu") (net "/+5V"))
 (segment (start 85.75 77.25) (end 85.75 80) (width 0.5) (layer "F.Cu") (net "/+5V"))
 (via (at 85.3 76.7) (size 0.6) (drill 0.3) (layers "F.Cu" "B.Cu") (free yes) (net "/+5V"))
 (segment (start 85.3 76.7) (end 85.3 72.73) (width 0.5) (layer "B.Cu") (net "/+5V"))
 (segment (start 85.3 72.73) (end 85.83 72.2) (width 0.5) (layer "B.Cu") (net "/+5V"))
 (segment (start 88.29 77.19) (end 88.29 80) (width 0.5) (layer "F.Cu") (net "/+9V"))
 (segment (start 87.8 76.7) (end 88.29 77.19) (width 0.5) (layer "F.Cu") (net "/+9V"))
 (via (at 87.8 76.7) (size 0.6) (drill 0.3) (layers "F.Cu" "B.Cu") (free yes) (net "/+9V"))
 (segment (start 87.8 76.7) (end 88.37 76.13) (width 0.5) (layer "B.Cu") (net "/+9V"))
 (segment (start 88.37 76.13) (end 88.37 72.2) (width 0.5) (layer "B.Cu") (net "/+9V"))
 (segment (start 95.4 76.7) (end 95.91 77.21) (width 0.5) (layer "F.Cu") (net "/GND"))
 (segment (start 113.69 77.19) (end 113.69 80) (width 0.5) (layer "F.Cu") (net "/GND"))
 (segment (start 113.3 76.8) (end 113.69 77.19) (width 0.5) (layer "F.Cu") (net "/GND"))
 (segment (start 113.3 76.7) (end 113.3 76.8) (width 0.5) (layer "F.Cu") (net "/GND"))
 (segment (start 95.91 77.21) (end 95.91 80) (width 0.5) (layer "F.Cu") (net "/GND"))
 (segment (start 93.37 77.17) (end 93.37 80) (width 0.5) (layer "F.Cu") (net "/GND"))
 (segment (start 92.9 76.7) (end 93.37 77.17) (width 0.5) (layer "F.Cu") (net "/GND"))
 (via (at 113.3 76.7) (size 0.6) (drill 0.3) (layers "F.Cu" "B.Cu") (free yes) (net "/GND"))
 (via (at 95.4 76.7) (size 0.6) (drill 0.3) (layers "F.Cu" "B.Cu") (free yes) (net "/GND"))
 (via (at 92.9 76.7) (size 0.6) (drill 0.3) (layers "F.Cu" "B.Cu") (free yes) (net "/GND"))
 (segment (start 92.9 76.7) (end 92.9 72.75) (width 0.5) (layer "B.Cu") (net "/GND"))
 (segment (start 92.9 72.75) (end 93.45 72.2) (width 0.5) (layer "B.Cu") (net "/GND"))
 (segment (start 95.4 72.79) (end 95.99 72.2) (width 0.5) (layer "B.Cu") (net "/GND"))
 (segment (start 113.3 76.7) (end 113.3 72.67) (width 0.5) (layer "B.Cu") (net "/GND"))
 (segment (start 113.3 72.67) (end 113.77 72.2) (width 0.5) (layer "B.Cu") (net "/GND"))
 (segment (start 95.4 76.7) (end 95.4 72.79) (width 0.5) (layer "B.Cu") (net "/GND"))
 (segment (start 98 76.7) (end 98.45 77.15) (width 0.5) (layer "F.Cu") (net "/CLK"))
 (segment (start 98.45 77.15) (end 98.45 80) (width 0.5) (layer "F.Cu") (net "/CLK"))
 (via (at 98 76.7) (size 0.6) (drill 0.3) (layers "F.Cu" "B.Cu") (free yes) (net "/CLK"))
 (segment (start 98 76.7) (end 98 72.73) (width 0.5) (layer "B.Cu") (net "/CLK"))
 (segment (start 98 72.73) (end 98.53 72.2) (width 0.5) (layer "B.Cu") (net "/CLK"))
 (segment (start 100.99 77.19) (end 100.99 80) (width 0.5) (layer "F.Cu") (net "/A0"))
 (segment (start 100.5 76.7) (end 100.99 77.19) (width 0.5) (layer "F.Cu") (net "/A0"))
 (via (at 100.5 76.7) (size 0.6) (drill 0.3) (layers "F.Cu" "B.Cu") (free yes) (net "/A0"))
 (segment (start 100.5 72.77) (end 101.07 72.2) (width 0.5) (layer "B.Cu") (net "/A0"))
 (segment (start 100.5 76.7) (end 100.5 72.77) (width 0.5) (layer "B.Cu") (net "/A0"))
 (segment (start 103.1 76.7) (end 103.53 77.13) (width 0.5) (layer "F.Cu") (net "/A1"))
 (segment (start 103.53 77.13) (end 103.53 80) (width 0.5) (layer "F.Cu") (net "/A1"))
 (via (at 103.1 76.7) (size 0.6) (drill 0.3) (layers "F.Cu" "B.Cu") (free yes) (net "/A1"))
 (segment (start 103.1 72.71) (end 103.61 72.2) (width 0.5) (layer "B.Cu") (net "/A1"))
 (segment (start 103.1 76.7) (end 103.1 72.71) (width 0.5) (layer "B.Cu") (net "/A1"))
 (segment (start 105.6 76.7) (end 106.07 77.17) (width 0.5) (layer "F.Cu") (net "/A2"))
 (segment (start 106.07 77.17) (end 106.07 80) (width 0.5) (layer "F.Cu") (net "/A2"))
 (via (at 105.6 76.7) (size 0.6) (drill 0.3) (layers "F.Cu" "B.Cu") (free yes) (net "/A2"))
 (segment (start 105.6 72.75) (end 106.15 72.2) (width 0.5) (layer "B.Cu") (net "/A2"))
 (segment (start 105.6 76.7) (end 105.6 72.75) (width 0.5) (layer "B.Cu") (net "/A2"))
 (segment (start 108.2 76.7) (end 108.61 77.11) (width 0.5) (layer "F.Cu") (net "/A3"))
 (segment (start 108.61 77.11) (end 108.61 80) (width 0.5) (layer "F.Cu") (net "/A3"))
 (via (at 108.2 76.7) (size 0.6) (drill 0.3) (layers "F.Cu" "B.Cu") (free yes) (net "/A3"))
 (segment (start 108.2 72.69) (end 108.69 72.2) (width 0.5) (layer "B.Cu") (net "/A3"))
 (segment (start 108.2 76.7) (end 108.2 72.69) (width 0.5) (layer "B.Cu") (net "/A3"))
 (segment (start 110.7 76.7) (end 111.15 77.15) (width 0.5) (layer "F.Cu") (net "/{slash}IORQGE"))
 (segment (start 111.15 77.15) (end 111.15 80) (width 0.5) (layer "F.Cu") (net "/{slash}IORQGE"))
 (via (at 110.7 76.7) (size 0.6) (drill 0.3) (layers "F.Cu" "B.Cu") (free yes) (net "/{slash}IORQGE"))
 (segment (start 110.7 76.7) (end 110.7 72.73) (width 0.5) (layer "B.Cu") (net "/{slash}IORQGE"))
 (segment (start 110.7 72.73) (end 111.23 72.2) (width 0.5) (layer "B.Cu") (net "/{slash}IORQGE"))
 (segment (start 115.8 76.7) (end 116.23 77.13) (width 0.5) (layer "F.Cu") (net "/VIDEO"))
 (segment (start 116.23 77.13) (end 116.23 80) (width 0.5) (layer "F.Cu") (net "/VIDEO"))
 (via (at 115.8 76.7) (size 0.6) (drill 0.3) (layers "F.Cu" "B.Cu") (free yes) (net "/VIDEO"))
 (segment (start 115.8 72.71) (end 116.31 72.2) (width 0.5) (layer "B.Cu") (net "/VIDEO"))
 (segment (start 115.8 76.7) (end 115.8 72.71) (width 0.5) (layer "B.Cu") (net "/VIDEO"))
 (segment (start 118.77 77.07) (end 118.77 80) (width 0.5) (layer "F.Cu") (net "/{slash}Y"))
 (segment (start 118.4 76.7) (end 118.77 77.07) (width 0.5) (layer "F.Cu") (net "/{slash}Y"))
 (via (at 118.4 76.7) (size 0.6) (drill 0.3) (layers "F.Cu" "B.Cu") (free yes) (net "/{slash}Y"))
 (segment (start 118.4 72.65) (end 118.85 72.2) (width 0.5) (layer "B.Cu") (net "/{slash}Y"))
 (segment (start 118.4 76.7) (end 118.4 72.65) (width 0.5) (layer "B.Cu") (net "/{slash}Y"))
 (segment (start 121.31 77.11) (end 121.31 80) (width 0.5) (layer "F.Cu") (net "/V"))
 (segment (start 120.9 76.7) (end 121.31 77.11) (width 0.5) (layer "F.Cu") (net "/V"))
 (via (at 120.9 76.7) (size 0.6) (drill 0.3) (layers "F.Cu" "B.Cu") (free yes) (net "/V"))
 (segment (start 120.9 72.69) (end 121.39 72.2) (width 0.5) (layer "B.Cu") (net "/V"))
 (segment (start 120.9 76.7) (end 120.9 72.69) (width 0.5) (layer "B.Cu") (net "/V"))
 (segment (start 123.85 77.05) (end 123.85 80) (width 0.5) (layer "F.Cu") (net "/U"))
 (segment (start 123.5 76.7) (end 123.85 77.05) (width 0.5) (layer "F.Cu") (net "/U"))
 (via (at 123.5 76.7) (size 0.6) (drill 0.3) (layers "F.Cu" "B.Cu") (free yes) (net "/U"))
 (segment (start 123.5 72.63) (end 123.93 72.2) (width 0.5) (layer "B.Cu") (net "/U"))
 (segment (start 123.5 76.7) (end 123.5 72.63) (width 0.5) (layer "B.Cu") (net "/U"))
 (segment (start 126 76.7) (end 126.39 77.09) (width 0.5) (layer "F.Cu") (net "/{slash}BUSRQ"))
 (segment (start 126.39 77.09) (end 126.39 80) (width 0.5) (layer "F.Cu") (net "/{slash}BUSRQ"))
 (via (at 126 76.7) (size 0.6) (drill 0.3) (layers "F.Cu" "B.Cu") (free yes) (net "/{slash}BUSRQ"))
 (segment (start 126 72.67) (end 126.47 72.2) (width 0.5) (layer "B.Cu") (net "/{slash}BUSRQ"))
 (segment (start 126 76.7) (end 126 72.67) (width 0.5) (layer "B.Cu") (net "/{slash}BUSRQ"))
 (segment (start 128.93 77.03) (end 128.93 80) (width 0.5) (layer "F.Cu") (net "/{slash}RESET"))
 (segment (start 128.6 76.7) (end 128.93 77.03) (width 0.5) (layer "F.Cu") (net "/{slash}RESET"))
 (via (at 128.6 76.7) (size 0.6) (drill 0.3) (layers "F.Cu" "B.Cu") (free yes) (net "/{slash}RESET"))
 (segment (start 128.6 72.61) (end 129.01 72.2) (width 0.5) (layer "B.Cu") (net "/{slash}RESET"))
 (segment (start 128.6 76.7) (end 128.6 72.61) (width 0.5) (layer "B.Cu") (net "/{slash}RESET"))
 (segment (start 131.47 77.07) (end 131.47 80) (width 0.5) (layer "F.Cu") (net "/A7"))
 (segment (start 131.1 76.7) (end 131.47 77.07) (width 0.5) (layer "F.Cu") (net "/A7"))
 (via (at 131.1 76.7) (size 0.6) (drill 0.3) (layers "F.Cu" "B.Cu") (free yes) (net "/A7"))
 (segment (start 131.1 76.7) (end 131.1 72.65) (width 0.5) (layer "B.Cu") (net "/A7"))
 (segment (start 131.1 72.65) (end 131.55 72.2) (width 0.5) (layer "B.Cu") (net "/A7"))
 (segment (start 134.01 77.21) (end 134.01 80) (width 0.5) (layer "F.Cu") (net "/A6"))
 (segment (start 133.5 76.7) (end 134.01 77.21) (width 0.5) (layer "F.Cu") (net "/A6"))
 (via (at 133.5 76.7) (size 0.6) (drill 0.3) (layers "F.Cu" "B.Cu") (free yes) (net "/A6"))
 (segment (start 133.5 76.7) (end 133.5 72.79) (width 0.5) (layer "B.Cu") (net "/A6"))
 (segment (start 133.5 72.79) (end 134.09 72.2) (width 0.5) (layer "B.Cu") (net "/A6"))
 (segment (start 136.1 76.7) (end 136.55 77.15) (width 0.5) (layer "F.Cu") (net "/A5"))
 (segment (start 136.55 77.15) (end 136.55 80) (width 0.5) (layer "F.Cu") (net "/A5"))
 (via (at 136.1 76.7) (size 0.6) (drill 0.3) (layers "F.Cu" "B.Cu") (free yes) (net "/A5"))
 (segment (start 136.1 76.7) (end 136.1 72.73) (width 0.5) (layer "B.Cu") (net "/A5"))
 (segment (start 136.1 72.73) (end 136.63 72.2) (width 0.5) (layer "B.Cu") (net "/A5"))
 (segment (start 138.6 76.7) (end 139.09 77.19) (width 0.5) (layer "F.Cu") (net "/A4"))
 (segment (start 139.09 77.19) (end 139.09 80) (width 0.5) (layer "F.Cu") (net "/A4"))
 (via (at 138.6 76.7) (size 0.6) (drill 0.3) (layers "F.Cu" "B.Cu") (free yes) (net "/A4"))
 (segment (start 138.6 76.7) (end 138.6 72.77) (width 0.5) (layer "B.Cu") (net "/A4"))
 (segment (start 138.6 72.77) (end 139.17 72.2) (width 0.5) (layer "B.Cu") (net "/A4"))
 (segment (start 141.2 76.7) (end 141.63 77.13) (width 0.5) (layer "F.Cu") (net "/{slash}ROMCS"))
 (segment (start 141.63 77.13) (end 141.63 80) (width 0.5) (layer "F.Cu") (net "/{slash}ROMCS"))
 (via (at 141.2 76.7) (size 0.6) (drill 0.3) (layers "F.Cu" "B.Cu") (free yes) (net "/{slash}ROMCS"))
 (segment (start 141.2 76.7) (end 141.2 72.71) (width 0.5) (layer "B.Cu") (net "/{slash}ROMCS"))
 (segment (start 141.2 72.71) (end 141.71 72.2) (width 0.5) (layer "B.Cu") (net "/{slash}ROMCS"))
 (segment (start 144.17 77.17) (end 144.17 80) (width 0.5) (layer "F.Cu") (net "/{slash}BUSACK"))
 (segment (start 143.7 76.7) (end 144.17 77.17) (width 0.5) (layer "F.Cu") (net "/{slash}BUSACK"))
 (via (at 143.7 76.7) (size 0.6) (drill 0.3) (layers "F.Cu" "B.Cu") (free yes) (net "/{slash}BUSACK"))
 (segment (start 143.7 76.7) (end 143.7 72.75) (width 0.5) (layer "B.Cu") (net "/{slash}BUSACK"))
 (segment (start 143.7 72.75) (end 144.25 72.2) (width 0.5) (layer "B.Cu") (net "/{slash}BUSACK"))
 (segment (start 146.71 77.11) (end 146.71 80) (width 0.5) (layer "F.Cu") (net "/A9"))
 (segment (start 146.3 76.7) (end 146.71 77.11) (width 0.5) (layer "F.Cu") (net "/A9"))
 (via (at 146.3 76.7) (size 0.6) (drill 0.3) (layers "F.Cu" "B.Cu") (free yes) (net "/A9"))
 (segment (start 146.3 76.7) (end 146.3 72.69) (width 0.5) (layer "B.Cu") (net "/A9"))
 (segment (start 146.3 72.69) (end 146.79 72.2) (width 0.5) (layer "B.Cu") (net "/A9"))
 (segment (start 149.25 77.15) (end 149.25 80) (width 0.5) (layer "F.Cu") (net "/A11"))
 (segment (start 148.8 76.7) (end 149.25 77.15) (width 0.5) (layer "F.Cu") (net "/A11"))
 (via (at 148.8 76.7) (size 0.6) (drill 0.3) (layers "F.Cu" "B.Cu") (free yes) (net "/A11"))
 (segment (start 148.8 76.7) (end 149.33 76.17) (width 0.5) (layer "B.Cu") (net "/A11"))
 (segment (start 149.33 76.17) (end 149.33 72.2) (width 0.5) (layer "B.Cu") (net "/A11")))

